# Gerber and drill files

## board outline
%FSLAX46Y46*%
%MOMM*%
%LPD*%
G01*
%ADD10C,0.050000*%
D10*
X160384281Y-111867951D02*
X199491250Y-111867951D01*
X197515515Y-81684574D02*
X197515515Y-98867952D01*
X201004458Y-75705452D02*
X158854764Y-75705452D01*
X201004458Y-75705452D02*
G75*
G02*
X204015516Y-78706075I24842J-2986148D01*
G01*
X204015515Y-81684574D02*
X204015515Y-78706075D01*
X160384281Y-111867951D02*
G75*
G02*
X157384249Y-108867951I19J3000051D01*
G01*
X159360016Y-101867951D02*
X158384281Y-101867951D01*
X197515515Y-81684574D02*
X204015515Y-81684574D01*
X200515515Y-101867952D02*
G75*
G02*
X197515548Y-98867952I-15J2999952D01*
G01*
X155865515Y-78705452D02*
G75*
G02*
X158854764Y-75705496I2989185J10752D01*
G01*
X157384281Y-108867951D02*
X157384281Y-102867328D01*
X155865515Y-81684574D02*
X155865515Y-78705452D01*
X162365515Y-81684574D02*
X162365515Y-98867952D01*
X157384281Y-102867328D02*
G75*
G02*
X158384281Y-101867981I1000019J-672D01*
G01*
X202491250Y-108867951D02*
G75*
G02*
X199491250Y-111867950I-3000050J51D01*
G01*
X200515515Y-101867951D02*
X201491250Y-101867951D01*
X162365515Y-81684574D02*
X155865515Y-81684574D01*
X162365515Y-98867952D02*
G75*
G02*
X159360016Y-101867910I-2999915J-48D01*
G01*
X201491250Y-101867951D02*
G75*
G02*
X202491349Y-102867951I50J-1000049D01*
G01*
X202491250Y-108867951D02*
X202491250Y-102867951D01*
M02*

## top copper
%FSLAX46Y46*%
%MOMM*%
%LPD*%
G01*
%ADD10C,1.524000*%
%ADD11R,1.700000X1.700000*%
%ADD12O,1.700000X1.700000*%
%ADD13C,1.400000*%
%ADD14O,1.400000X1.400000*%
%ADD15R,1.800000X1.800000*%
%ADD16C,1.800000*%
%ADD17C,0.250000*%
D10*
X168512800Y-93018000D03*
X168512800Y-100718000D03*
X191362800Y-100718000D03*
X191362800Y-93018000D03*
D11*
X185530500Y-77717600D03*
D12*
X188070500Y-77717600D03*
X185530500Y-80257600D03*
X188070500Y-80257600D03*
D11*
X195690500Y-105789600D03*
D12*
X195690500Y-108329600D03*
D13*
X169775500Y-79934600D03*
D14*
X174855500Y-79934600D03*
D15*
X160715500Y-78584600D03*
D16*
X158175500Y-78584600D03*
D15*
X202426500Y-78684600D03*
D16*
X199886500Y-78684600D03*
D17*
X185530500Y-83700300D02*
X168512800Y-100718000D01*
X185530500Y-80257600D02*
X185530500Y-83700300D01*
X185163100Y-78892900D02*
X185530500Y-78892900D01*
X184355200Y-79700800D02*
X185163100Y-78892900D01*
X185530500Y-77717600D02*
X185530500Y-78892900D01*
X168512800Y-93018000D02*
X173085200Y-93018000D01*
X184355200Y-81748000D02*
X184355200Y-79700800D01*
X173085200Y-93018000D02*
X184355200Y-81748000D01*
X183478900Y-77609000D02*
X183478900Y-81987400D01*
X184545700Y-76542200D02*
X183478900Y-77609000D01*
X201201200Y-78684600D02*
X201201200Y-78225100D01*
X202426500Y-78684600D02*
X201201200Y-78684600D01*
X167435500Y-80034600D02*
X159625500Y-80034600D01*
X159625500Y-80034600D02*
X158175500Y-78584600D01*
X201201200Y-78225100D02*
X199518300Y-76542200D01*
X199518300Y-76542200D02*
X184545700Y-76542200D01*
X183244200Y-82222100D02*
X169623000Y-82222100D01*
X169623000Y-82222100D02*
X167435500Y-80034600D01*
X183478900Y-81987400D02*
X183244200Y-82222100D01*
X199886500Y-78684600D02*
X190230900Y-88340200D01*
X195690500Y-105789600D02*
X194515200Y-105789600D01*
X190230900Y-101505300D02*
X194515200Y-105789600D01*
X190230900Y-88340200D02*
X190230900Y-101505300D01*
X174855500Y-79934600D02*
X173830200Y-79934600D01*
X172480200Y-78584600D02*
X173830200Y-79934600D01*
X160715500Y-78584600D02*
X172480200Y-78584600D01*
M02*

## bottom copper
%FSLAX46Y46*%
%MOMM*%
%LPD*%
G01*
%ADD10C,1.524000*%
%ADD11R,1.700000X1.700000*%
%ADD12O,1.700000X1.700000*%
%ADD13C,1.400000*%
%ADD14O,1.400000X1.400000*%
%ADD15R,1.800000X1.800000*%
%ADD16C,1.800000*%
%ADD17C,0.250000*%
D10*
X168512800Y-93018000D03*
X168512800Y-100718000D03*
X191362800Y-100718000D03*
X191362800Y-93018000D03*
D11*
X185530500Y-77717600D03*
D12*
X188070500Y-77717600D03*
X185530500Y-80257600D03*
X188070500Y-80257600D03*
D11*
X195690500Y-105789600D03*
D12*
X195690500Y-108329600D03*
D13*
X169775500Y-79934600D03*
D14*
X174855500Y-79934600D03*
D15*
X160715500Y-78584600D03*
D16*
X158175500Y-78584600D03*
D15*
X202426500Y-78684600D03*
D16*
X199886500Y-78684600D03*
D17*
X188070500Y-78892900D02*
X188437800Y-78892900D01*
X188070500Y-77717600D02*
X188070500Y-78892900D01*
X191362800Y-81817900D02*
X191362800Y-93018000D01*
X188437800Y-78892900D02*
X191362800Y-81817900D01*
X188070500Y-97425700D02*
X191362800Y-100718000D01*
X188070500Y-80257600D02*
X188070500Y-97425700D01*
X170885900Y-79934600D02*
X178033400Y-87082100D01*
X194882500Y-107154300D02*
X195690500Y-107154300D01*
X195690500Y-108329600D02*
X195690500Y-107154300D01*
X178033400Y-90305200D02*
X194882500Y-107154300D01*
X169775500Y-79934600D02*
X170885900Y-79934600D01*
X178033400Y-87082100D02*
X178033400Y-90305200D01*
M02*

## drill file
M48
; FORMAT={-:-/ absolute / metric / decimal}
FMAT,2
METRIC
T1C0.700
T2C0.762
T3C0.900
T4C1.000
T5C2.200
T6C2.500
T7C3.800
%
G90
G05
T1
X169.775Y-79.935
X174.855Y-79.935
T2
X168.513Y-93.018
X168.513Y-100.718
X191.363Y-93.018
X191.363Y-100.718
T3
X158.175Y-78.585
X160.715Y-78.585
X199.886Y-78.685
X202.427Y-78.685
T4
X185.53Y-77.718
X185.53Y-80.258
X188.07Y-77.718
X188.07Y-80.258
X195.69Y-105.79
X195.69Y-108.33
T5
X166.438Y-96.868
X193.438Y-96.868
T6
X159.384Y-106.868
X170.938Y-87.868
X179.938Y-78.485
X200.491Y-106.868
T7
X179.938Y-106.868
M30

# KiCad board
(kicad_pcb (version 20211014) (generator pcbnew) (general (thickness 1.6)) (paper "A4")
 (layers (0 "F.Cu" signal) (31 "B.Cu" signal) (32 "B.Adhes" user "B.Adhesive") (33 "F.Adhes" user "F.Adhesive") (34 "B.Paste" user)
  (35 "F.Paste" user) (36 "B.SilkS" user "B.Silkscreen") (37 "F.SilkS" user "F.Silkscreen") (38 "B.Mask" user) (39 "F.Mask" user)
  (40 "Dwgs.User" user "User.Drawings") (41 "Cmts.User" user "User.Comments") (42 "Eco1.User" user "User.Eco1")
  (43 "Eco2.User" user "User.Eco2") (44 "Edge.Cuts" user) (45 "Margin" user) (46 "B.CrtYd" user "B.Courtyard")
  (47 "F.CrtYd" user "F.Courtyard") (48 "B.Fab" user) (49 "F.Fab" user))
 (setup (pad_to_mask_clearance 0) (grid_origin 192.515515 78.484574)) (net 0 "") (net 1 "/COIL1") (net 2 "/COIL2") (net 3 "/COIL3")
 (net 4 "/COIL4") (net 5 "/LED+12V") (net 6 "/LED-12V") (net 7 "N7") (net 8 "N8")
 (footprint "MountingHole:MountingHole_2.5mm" (layer "F.Cu") (at 179.9378 78.4846)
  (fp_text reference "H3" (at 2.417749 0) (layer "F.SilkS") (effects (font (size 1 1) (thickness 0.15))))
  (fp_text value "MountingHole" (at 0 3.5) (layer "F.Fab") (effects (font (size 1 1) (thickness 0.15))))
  (pad "" np_thru_hole circle locked (at 0 0) (size 2.5 2.5) (drill 2.5) (layers *.Cu *.Mask)))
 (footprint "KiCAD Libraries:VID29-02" (layer "F.Cu") (at 180.1028 96.868)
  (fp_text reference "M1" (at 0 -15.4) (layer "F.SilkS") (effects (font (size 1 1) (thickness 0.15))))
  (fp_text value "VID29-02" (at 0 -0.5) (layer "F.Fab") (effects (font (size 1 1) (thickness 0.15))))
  (pad "" np_thru_hole circle locked (at -9.165 -9) (size 2.5 2.5) (drill 2.5) (layers *.Cu *.Mask))
  (pad "" np_thru_hole circle locked (at 13.335 0) (size 2.2 2.2) (drill 2.2) (layers *.Cu *.Mask))
  (pad "" np_thru_hole circle locked (at -0.165 10) (size 3.8 3.8) (drill 3.8) (layers *.Cu *.Mask))
  (pad "" np_thru_hole circle locked (at -13.665 0) (size 2.2 2.2) (drill 2.2) (layers *.Cu *.Mask))
  (pad "1" thru_hole circle locked (at -11.59 -3.85) (size 1.524 1.524) (drill 0.762) (layers *.Cu *.Mask) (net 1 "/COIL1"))
  (pad "2" thru_hole circle locked (at -11.59 3.85) (size 1.524 1.524) (drill 0.762) (layers *.Cu *.Mask) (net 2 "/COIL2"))
  (pad "3" thru_hole circle locked (at 11.26 3.85) (size 1.524 1.524) (drill 0.762) (layers *.Cu *.Mask) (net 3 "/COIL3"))
  (pad "4" thru_hole circle locked (at 11.26 -3.85) (size 1.524 1.524) (drill 0.762) (layers *.Cu *.Mask) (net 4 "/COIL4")))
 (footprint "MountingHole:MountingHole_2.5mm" (layer "F.Cu") (at 159.3843 106.868)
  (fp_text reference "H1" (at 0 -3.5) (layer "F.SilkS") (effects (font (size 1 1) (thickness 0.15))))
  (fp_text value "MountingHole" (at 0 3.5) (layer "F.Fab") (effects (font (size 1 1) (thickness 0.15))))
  (pad "" np_thru_hole circle locked (at 0 0) (size 2.5 2.5) (drill 2.5) (layers *.Cu *.Mask)))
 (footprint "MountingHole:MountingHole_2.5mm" (layer "F.Cu") (at 200.4913 106.868)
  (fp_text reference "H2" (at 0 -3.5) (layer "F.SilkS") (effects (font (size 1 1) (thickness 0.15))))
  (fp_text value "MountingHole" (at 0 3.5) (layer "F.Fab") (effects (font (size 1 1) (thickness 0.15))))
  (pad "" np_thru_hole circle locked (at 0 0) (size 2.5 2.5) (drill 2.5) (layers *.Cu *.Mask)))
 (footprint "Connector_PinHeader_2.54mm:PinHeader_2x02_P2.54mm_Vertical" (layer "F.Cu") (at 185.5305 77.7176)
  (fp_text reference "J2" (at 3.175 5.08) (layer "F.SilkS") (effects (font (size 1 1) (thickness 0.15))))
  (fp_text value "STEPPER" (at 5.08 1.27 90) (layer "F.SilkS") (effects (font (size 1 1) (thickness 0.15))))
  (pad "1" thru_hole rect locked (at 0 0) (size 1.7 1.7) (drill 1) (layers *.Cu *.Mask) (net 1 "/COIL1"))
  (pad "2" thru_hole oval locked (at 2.54 0) (size 1.7 1.7) (drill 1) (layers *.Cu *.Mask) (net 4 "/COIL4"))
  (pad "3" thru_hole oval locked (at 0 2.54) (size 1.7 1.7) (drill 1) (layers *.Cu *.Mask) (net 2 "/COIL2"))
  (pad "4" thru_hole oval locked (at 2.54 2.54) (size 1.7 1.7) (drill 1) (layers *.Cu *.Mask) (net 3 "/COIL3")))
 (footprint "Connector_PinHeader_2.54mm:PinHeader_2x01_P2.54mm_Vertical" (layer "F.Cu") (at 195.6905 105.7896 -90)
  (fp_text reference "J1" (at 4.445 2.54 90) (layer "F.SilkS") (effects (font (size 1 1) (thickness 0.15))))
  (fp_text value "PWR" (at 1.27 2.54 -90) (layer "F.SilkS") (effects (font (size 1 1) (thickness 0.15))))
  (pad "1" thru_hole rect locked (at 0 0 270) (size 1.7 1.7) (drill 1) (layers *.Cu *.Mask) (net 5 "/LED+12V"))
  (pad "2" thru_hole oval locked (at 2.54 0 270) (size 1.7 1.7) (drill 1) (layers *.Cu *.Mask) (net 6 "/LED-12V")))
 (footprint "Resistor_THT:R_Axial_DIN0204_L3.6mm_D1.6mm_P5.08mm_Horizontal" (layer "F.Cu") (at 169.7755 79.9346)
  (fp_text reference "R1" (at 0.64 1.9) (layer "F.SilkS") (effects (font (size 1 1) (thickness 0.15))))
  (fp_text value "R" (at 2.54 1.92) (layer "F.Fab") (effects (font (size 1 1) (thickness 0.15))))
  (pad "1" thru_hole circle (at 0 0) (size 1.4 1.4) (drill 0.7) (layers *.Cu *.Mask) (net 6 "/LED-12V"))
  (pad "2" thru_hole oval (at 5.08 0) (size 1.4 1.4) (drill 0.7) (layers *.Cu *.Mask) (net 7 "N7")))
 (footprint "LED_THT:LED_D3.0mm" (layer "B.Cu") (at 160.7155 78.5846 180)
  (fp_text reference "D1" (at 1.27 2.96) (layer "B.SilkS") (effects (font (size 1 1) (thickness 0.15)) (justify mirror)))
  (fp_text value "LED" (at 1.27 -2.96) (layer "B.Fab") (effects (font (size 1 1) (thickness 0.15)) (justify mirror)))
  (pad "1" thru_hole rect (at 0 0 180) (size 1.8 1.8) (drill 0.9) (layers *.Cu *.Mask) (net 7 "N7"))
  (pad "2" thru_hole circle (at 2.54 0 180) (size 1.8 1.8) (drill 0.9) (layers *.Cu *.Mask) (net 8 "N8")))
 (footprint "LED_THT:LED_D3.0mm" (layer "B.Cu") (at 202.4265 78.6846 180)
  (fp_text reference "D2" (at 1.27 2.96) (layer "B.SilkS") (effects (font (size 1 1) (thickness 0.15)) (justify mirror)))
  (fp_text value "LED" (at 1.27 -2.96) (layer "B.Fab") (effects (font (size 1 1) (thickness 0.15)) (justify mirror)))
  (pad "1" thru_hole rect (at 0 0 180) (size 1.8 1.8) (drill 0.9) (layers *.Cu *.Mask) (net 8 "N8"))
  (pad "2" thru_hole circle (at 2.54 0 180) (size 1.8 1.8) (drill 0.9) (layers *.Cu *.Mask) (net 5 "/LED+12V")))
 (gr_line (start 160.384281 111.867951) (end 199.49125 111.867951) (layer "Edge.Cuts") (width 0.05))
 (gr_line (start 197.515515 81.684574) (end 197.515515 98.867952) (layer "Edge.Cuts") (width 0.05))
 (gr_line (start 201.004458 75.705452) (end 158.854764 75.705452) (layer "Edge.Cuts") (width 0.05))
 (gr_arc (start 201.004458 75.705452) (mid 203.137237 76.576331) (end 204.015515 78.706075) (layer "Edge.Cuts") (width 0.05))
 (gr_line (start 204.015515 81.684574) (end 204.015515 78.706075) (layer "Edge.Cuts") (width 0.05))
 (gr_arc (start 160.384281 111.867951) (mid 158.262961 110.989271) (end 157.384281 108.867951) (layer "Edge.Cuts") (width 0.05))
 (gr_line (start 159.360016 101.867951) (end 158.384281 101.867951) (layer "Edge.Cuts") (width 0.05))
 (gr_line (start 197.515515 81.684574) (end 204.015515 81.684574) (layer "Edge.Cuts") (width 0.05))
 (gr_arc (start 200.515515 101.867952) (mid 198.394195 100.989272) (end 197.515515 98.867952) (layer "Edge.Cuts") (width 0.05))
 (gr_arc (start 155.865515 78.705452) (mid 156.73723 76.584781) (end 158.854764 75.705452) (layer "Edge.Cuts") (width 0.05))
 (gr_line (start 157.384281 108.867951) (end 157.384281 102.867328) (layer "Edge.Cuts") (width 0.05))
 (gr_line (start 155.865515 81.684574) (end 155.865515 78.705452) (layer "Edge.Cuts") (width 0.05))
 (gr_line (start 162.365515 81.684574) (end 162.365515 98.867952) (layer "Edge.Cuts") (width 0.05))
 (gr_arc (start 157.384281 102.867328) (mid 157.677399 102.160628) (end 158.384281 101.867951) (layer "Edge.Cuts") (width 0.05))
 (gr_arc (start 202.49125 108.867951) (mid 201.61257 110.989271) (end 199.49125 111.867951) (layer "Edge.Cuts") (width 0.05))
 (gr_line (start 200.515515 101.867951) (end 201.49125 101.867951) (layer "Edge.Cuts") (width 0.05))
 (gr_line (start 162.365515 81.684574) (end 155.865515 81.684574) (layer "Edge.Cuts") (width 0.05))
 (gr_arc (start 162.365515 98.867952) (mid 161.484904 100.991231) (end 159.360016 101.867951) (layer "Edge.Cuts") (width 0.05))
 (gr_arc (start 201.49125 101.867951) (mid 202.198357 102.160844) (end 202.49125 102.867951) (layer "Edge.Cuts") (width 0.05))
 (gr_line (start 202.49125 108.867951) (end 202.49125 102.867951) (layer "Edge.Cuts") (width 0.05))
 (segment (start 185.5305 83.7003) (end 168.5128 100.718) (width 0.25) (layer "F.Cu") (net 2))
 (segment (start 185.5305 80.2576) (end 185.5305 83.7003) (width 0.25) (layer "F.Cu") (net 2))
 (segment (start 185.1631 78.8929) (end 185.5305 78.8929) (width 0.25) (layer "F.Cu") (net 1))
 (segment (start 184.3552 79.7008) (end 185.1631 78.8929) (width 0.25) (layer "F.Cu") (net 1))
 (segment (start 185.5305 77.7176) (end 185.5305 78.8929) (width 0.25) (layer "F.Cu") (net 1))
 (segment (start 168.5128 93.018) (end 173.0852 93.018) (width 0.25) (layer "F.Cu") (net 1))
 (segment (start 184.3552 81.748) (end 184.3552 79.7008) (width 0.25) (layer "F.Cu") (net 1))
 (segment (start 173.0852 93.018) (end 184.3552 81.748) (width 0.25) (layer "F.Cu") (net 1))
 (segment (start 188.0705 78.8929) (end 188.4378 78.8929) (width 0.25) (layer "B.Cu") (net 4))
 (segment (start 188.0705 77.7176) (end 188.0705 78.8929) (width 0.25) (layer "B.Cu") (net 4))
 (segment (start 191.3628 81.8179) (end 191.3628 93.018) (width 0.25) (layer "B.Cu") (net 4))
 (segment (start 188.4378 78.8929) (end 191.3628 81.8179) (width 0.25) (layer "B.Cu") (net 4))
 (segment (start 188.0705 97.4257) (end 191.3628 100.718) (width 0.25) (layer "B.Cu") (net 3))
 (segment (start 188.0705 80.2576) (end 188.0705 97.4257) (width 0.25) (layer "B.Cu") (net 3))
 (segment (start 183.4789 77.609) (end 183.4789 81.9874) (width 0.25) (layer "F.Cu") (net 8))
 (segment (start 184.5457 76.5422) (end 183.4789 77.609) (width 0.25) (layer "F.Cu") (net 8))
 (segment (start 201.2012 78.6846) (end 201.2012 78.2251) (width 0.25) (layer "F.Cu") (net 8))
 (segment (start 202.4265 78.6846) (end 201.2012 78.6846) (width 0.25) (layer "F.Cu") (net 8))
 (segment (start 167.4355 80.0346) (end 159.6255 80.0346) (width 0.25) (layer "F.Cu") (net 8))
 (segment (start 159.6255 80.0346) (end 158.1755 78.5846) (width 0.25) (layer "F.Cu") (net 8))
 (segment (start 201.2012 78.2251) (end 199.5183 76.5422) (width 0.25) (layer "F.Cu") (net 8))
 (segment (start 199.5183 76.5422) (end 184.5457 76.5422) (width 0.25) (layer "F.Cu") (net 8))
 (segment (start 183.2442 82.2221) (end 169.623 82.2221) (width 0.25) (layer "F.Cu") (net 8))
 (segment (start 169.623 82.2221) (end 167.4355 80.0346) (width 0.25) (layer "F.Cu") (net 8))
 (segment (start 183.4789 81.9874) (end 183.2442 82.2221) (width 0.25) (layer "F.Cu") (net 8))
 (segment (start 199.8865 78.6846) (end 190.2309 88.3402) (width 0.25) (layer "F.Cu") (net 5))
 (segment (start 195.6905 105.7896) (end 194.5152 105.7896) (width 0.25) (layer "F.Cu") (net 5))
 (segment (start 190.2309 101.5053) (end 194.5152 105.7896) (width 0.25) (layer "F.Cu") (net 5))
 (segment (start 190.2309 88.3402) (end 190.2309 101.5053) (width 0.25) (layer "F.Cu") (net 5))
 (segment (start 170.8859 79.9346) (end 178.0334 87.0821) (width 0.25) (layer "B.Cu") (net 6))
 (segment (start 194.8825 107.1543) (end 195.6905 107.1543) (width 0.25) (layer "B.Cu") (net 6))
 (segment (start 195.6905 108.3296) (end 195.6905 107.1543) (width 0.25) (layer "B.Cu") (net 6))
 (segment (start 178.0334 90.3052) (end 194.8825 107.1543) (width 0.25) (layer "B.Cu") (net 6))
 (segment (start 169.7755 79.9346) (end 170.8859 79.9346) (width 0.25) (layer "B.Cu") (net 6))
 (segment (start 178.0334 87.0821) (end 178.0334 90.3052) (width 0.25) (layer "B.Cu") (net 6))
 (segment (start 174.8555 79.9346) (end 173.8302 79.9346) (width 0.25) (layer "F.Cu") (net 7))
 (segment (start 172.4802 78.5846) (end 173.8302 79.9346) (width 0.25) (layer "F.Cu") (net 7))
 (segment (start 160.7155 78.5846) (end 172.4802 78.5846) (width 0.25) (layer "F.Cu") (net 7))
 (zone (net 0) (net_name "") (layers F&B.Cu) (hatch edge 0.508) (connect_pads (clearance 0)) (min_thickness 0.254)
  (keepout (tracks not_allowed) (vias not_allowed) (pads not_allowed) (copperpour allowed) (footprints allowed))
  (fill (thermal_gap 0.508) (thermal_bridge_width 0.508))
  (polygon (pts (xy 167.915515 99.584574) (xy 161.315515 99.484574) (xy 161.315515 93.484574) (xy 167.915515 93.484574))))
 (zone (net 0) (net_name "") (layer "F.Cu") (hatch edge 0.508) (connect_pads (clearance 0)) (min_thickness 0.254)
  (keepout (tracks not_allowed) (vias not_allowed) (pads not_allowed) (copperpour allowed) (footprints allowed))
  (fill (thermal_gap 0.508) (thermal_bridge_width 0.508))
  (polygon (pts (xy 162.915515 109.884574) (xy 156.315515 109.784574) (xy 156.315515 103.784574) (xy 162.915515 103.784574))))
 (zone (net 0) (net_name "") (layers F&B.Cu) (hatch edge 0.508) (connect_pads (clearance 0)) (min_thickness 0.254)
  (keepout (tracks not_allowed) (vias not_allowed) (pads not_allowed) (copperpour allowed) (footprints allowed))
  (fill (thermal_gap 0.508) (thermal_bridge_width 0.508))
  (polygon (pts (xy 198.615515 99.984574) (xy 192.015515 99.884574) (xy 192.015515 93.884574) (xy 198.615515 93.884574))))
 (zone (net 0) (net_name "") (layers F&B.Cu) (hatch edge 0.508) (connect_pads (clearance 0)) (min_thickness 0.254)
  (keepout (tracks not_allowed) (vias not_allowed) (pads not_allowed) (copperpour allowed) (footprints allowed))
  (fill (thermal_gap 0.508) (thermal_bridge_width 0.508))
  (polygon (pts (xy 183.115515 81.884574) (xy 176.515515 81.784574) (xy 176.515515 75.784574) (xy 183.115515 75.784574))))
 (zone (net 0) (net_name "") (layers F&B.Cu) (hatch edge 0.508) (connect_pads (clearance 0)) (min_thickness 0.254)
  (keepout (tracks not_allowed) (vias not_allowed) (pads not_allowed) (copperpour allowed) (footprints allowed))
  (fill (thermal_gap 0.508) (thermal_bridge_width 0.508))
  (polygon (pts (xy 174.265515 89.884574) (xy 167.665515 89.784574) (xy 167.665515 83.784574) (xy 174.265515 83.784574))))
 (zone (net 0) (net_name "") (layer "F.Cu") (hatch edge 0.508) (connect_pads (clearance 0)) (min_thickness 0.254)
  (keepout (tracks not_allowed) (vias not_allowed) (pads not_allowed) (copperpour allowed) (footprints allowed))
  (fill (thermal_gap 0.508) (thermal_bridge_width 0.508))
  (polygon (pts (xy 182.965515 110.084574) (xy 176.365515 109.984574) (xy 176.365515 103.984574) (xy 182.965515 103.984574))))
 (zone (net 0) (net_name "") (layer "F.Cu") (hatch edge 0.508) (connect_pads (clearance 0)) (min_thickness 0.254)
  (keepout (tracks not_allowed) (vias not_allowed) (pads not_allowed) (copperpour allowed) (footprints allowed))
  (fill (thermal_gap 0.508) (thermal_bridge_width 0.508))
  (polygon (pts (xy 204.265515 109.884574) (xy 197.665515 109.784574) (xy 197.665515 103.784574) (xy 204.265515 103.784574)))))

